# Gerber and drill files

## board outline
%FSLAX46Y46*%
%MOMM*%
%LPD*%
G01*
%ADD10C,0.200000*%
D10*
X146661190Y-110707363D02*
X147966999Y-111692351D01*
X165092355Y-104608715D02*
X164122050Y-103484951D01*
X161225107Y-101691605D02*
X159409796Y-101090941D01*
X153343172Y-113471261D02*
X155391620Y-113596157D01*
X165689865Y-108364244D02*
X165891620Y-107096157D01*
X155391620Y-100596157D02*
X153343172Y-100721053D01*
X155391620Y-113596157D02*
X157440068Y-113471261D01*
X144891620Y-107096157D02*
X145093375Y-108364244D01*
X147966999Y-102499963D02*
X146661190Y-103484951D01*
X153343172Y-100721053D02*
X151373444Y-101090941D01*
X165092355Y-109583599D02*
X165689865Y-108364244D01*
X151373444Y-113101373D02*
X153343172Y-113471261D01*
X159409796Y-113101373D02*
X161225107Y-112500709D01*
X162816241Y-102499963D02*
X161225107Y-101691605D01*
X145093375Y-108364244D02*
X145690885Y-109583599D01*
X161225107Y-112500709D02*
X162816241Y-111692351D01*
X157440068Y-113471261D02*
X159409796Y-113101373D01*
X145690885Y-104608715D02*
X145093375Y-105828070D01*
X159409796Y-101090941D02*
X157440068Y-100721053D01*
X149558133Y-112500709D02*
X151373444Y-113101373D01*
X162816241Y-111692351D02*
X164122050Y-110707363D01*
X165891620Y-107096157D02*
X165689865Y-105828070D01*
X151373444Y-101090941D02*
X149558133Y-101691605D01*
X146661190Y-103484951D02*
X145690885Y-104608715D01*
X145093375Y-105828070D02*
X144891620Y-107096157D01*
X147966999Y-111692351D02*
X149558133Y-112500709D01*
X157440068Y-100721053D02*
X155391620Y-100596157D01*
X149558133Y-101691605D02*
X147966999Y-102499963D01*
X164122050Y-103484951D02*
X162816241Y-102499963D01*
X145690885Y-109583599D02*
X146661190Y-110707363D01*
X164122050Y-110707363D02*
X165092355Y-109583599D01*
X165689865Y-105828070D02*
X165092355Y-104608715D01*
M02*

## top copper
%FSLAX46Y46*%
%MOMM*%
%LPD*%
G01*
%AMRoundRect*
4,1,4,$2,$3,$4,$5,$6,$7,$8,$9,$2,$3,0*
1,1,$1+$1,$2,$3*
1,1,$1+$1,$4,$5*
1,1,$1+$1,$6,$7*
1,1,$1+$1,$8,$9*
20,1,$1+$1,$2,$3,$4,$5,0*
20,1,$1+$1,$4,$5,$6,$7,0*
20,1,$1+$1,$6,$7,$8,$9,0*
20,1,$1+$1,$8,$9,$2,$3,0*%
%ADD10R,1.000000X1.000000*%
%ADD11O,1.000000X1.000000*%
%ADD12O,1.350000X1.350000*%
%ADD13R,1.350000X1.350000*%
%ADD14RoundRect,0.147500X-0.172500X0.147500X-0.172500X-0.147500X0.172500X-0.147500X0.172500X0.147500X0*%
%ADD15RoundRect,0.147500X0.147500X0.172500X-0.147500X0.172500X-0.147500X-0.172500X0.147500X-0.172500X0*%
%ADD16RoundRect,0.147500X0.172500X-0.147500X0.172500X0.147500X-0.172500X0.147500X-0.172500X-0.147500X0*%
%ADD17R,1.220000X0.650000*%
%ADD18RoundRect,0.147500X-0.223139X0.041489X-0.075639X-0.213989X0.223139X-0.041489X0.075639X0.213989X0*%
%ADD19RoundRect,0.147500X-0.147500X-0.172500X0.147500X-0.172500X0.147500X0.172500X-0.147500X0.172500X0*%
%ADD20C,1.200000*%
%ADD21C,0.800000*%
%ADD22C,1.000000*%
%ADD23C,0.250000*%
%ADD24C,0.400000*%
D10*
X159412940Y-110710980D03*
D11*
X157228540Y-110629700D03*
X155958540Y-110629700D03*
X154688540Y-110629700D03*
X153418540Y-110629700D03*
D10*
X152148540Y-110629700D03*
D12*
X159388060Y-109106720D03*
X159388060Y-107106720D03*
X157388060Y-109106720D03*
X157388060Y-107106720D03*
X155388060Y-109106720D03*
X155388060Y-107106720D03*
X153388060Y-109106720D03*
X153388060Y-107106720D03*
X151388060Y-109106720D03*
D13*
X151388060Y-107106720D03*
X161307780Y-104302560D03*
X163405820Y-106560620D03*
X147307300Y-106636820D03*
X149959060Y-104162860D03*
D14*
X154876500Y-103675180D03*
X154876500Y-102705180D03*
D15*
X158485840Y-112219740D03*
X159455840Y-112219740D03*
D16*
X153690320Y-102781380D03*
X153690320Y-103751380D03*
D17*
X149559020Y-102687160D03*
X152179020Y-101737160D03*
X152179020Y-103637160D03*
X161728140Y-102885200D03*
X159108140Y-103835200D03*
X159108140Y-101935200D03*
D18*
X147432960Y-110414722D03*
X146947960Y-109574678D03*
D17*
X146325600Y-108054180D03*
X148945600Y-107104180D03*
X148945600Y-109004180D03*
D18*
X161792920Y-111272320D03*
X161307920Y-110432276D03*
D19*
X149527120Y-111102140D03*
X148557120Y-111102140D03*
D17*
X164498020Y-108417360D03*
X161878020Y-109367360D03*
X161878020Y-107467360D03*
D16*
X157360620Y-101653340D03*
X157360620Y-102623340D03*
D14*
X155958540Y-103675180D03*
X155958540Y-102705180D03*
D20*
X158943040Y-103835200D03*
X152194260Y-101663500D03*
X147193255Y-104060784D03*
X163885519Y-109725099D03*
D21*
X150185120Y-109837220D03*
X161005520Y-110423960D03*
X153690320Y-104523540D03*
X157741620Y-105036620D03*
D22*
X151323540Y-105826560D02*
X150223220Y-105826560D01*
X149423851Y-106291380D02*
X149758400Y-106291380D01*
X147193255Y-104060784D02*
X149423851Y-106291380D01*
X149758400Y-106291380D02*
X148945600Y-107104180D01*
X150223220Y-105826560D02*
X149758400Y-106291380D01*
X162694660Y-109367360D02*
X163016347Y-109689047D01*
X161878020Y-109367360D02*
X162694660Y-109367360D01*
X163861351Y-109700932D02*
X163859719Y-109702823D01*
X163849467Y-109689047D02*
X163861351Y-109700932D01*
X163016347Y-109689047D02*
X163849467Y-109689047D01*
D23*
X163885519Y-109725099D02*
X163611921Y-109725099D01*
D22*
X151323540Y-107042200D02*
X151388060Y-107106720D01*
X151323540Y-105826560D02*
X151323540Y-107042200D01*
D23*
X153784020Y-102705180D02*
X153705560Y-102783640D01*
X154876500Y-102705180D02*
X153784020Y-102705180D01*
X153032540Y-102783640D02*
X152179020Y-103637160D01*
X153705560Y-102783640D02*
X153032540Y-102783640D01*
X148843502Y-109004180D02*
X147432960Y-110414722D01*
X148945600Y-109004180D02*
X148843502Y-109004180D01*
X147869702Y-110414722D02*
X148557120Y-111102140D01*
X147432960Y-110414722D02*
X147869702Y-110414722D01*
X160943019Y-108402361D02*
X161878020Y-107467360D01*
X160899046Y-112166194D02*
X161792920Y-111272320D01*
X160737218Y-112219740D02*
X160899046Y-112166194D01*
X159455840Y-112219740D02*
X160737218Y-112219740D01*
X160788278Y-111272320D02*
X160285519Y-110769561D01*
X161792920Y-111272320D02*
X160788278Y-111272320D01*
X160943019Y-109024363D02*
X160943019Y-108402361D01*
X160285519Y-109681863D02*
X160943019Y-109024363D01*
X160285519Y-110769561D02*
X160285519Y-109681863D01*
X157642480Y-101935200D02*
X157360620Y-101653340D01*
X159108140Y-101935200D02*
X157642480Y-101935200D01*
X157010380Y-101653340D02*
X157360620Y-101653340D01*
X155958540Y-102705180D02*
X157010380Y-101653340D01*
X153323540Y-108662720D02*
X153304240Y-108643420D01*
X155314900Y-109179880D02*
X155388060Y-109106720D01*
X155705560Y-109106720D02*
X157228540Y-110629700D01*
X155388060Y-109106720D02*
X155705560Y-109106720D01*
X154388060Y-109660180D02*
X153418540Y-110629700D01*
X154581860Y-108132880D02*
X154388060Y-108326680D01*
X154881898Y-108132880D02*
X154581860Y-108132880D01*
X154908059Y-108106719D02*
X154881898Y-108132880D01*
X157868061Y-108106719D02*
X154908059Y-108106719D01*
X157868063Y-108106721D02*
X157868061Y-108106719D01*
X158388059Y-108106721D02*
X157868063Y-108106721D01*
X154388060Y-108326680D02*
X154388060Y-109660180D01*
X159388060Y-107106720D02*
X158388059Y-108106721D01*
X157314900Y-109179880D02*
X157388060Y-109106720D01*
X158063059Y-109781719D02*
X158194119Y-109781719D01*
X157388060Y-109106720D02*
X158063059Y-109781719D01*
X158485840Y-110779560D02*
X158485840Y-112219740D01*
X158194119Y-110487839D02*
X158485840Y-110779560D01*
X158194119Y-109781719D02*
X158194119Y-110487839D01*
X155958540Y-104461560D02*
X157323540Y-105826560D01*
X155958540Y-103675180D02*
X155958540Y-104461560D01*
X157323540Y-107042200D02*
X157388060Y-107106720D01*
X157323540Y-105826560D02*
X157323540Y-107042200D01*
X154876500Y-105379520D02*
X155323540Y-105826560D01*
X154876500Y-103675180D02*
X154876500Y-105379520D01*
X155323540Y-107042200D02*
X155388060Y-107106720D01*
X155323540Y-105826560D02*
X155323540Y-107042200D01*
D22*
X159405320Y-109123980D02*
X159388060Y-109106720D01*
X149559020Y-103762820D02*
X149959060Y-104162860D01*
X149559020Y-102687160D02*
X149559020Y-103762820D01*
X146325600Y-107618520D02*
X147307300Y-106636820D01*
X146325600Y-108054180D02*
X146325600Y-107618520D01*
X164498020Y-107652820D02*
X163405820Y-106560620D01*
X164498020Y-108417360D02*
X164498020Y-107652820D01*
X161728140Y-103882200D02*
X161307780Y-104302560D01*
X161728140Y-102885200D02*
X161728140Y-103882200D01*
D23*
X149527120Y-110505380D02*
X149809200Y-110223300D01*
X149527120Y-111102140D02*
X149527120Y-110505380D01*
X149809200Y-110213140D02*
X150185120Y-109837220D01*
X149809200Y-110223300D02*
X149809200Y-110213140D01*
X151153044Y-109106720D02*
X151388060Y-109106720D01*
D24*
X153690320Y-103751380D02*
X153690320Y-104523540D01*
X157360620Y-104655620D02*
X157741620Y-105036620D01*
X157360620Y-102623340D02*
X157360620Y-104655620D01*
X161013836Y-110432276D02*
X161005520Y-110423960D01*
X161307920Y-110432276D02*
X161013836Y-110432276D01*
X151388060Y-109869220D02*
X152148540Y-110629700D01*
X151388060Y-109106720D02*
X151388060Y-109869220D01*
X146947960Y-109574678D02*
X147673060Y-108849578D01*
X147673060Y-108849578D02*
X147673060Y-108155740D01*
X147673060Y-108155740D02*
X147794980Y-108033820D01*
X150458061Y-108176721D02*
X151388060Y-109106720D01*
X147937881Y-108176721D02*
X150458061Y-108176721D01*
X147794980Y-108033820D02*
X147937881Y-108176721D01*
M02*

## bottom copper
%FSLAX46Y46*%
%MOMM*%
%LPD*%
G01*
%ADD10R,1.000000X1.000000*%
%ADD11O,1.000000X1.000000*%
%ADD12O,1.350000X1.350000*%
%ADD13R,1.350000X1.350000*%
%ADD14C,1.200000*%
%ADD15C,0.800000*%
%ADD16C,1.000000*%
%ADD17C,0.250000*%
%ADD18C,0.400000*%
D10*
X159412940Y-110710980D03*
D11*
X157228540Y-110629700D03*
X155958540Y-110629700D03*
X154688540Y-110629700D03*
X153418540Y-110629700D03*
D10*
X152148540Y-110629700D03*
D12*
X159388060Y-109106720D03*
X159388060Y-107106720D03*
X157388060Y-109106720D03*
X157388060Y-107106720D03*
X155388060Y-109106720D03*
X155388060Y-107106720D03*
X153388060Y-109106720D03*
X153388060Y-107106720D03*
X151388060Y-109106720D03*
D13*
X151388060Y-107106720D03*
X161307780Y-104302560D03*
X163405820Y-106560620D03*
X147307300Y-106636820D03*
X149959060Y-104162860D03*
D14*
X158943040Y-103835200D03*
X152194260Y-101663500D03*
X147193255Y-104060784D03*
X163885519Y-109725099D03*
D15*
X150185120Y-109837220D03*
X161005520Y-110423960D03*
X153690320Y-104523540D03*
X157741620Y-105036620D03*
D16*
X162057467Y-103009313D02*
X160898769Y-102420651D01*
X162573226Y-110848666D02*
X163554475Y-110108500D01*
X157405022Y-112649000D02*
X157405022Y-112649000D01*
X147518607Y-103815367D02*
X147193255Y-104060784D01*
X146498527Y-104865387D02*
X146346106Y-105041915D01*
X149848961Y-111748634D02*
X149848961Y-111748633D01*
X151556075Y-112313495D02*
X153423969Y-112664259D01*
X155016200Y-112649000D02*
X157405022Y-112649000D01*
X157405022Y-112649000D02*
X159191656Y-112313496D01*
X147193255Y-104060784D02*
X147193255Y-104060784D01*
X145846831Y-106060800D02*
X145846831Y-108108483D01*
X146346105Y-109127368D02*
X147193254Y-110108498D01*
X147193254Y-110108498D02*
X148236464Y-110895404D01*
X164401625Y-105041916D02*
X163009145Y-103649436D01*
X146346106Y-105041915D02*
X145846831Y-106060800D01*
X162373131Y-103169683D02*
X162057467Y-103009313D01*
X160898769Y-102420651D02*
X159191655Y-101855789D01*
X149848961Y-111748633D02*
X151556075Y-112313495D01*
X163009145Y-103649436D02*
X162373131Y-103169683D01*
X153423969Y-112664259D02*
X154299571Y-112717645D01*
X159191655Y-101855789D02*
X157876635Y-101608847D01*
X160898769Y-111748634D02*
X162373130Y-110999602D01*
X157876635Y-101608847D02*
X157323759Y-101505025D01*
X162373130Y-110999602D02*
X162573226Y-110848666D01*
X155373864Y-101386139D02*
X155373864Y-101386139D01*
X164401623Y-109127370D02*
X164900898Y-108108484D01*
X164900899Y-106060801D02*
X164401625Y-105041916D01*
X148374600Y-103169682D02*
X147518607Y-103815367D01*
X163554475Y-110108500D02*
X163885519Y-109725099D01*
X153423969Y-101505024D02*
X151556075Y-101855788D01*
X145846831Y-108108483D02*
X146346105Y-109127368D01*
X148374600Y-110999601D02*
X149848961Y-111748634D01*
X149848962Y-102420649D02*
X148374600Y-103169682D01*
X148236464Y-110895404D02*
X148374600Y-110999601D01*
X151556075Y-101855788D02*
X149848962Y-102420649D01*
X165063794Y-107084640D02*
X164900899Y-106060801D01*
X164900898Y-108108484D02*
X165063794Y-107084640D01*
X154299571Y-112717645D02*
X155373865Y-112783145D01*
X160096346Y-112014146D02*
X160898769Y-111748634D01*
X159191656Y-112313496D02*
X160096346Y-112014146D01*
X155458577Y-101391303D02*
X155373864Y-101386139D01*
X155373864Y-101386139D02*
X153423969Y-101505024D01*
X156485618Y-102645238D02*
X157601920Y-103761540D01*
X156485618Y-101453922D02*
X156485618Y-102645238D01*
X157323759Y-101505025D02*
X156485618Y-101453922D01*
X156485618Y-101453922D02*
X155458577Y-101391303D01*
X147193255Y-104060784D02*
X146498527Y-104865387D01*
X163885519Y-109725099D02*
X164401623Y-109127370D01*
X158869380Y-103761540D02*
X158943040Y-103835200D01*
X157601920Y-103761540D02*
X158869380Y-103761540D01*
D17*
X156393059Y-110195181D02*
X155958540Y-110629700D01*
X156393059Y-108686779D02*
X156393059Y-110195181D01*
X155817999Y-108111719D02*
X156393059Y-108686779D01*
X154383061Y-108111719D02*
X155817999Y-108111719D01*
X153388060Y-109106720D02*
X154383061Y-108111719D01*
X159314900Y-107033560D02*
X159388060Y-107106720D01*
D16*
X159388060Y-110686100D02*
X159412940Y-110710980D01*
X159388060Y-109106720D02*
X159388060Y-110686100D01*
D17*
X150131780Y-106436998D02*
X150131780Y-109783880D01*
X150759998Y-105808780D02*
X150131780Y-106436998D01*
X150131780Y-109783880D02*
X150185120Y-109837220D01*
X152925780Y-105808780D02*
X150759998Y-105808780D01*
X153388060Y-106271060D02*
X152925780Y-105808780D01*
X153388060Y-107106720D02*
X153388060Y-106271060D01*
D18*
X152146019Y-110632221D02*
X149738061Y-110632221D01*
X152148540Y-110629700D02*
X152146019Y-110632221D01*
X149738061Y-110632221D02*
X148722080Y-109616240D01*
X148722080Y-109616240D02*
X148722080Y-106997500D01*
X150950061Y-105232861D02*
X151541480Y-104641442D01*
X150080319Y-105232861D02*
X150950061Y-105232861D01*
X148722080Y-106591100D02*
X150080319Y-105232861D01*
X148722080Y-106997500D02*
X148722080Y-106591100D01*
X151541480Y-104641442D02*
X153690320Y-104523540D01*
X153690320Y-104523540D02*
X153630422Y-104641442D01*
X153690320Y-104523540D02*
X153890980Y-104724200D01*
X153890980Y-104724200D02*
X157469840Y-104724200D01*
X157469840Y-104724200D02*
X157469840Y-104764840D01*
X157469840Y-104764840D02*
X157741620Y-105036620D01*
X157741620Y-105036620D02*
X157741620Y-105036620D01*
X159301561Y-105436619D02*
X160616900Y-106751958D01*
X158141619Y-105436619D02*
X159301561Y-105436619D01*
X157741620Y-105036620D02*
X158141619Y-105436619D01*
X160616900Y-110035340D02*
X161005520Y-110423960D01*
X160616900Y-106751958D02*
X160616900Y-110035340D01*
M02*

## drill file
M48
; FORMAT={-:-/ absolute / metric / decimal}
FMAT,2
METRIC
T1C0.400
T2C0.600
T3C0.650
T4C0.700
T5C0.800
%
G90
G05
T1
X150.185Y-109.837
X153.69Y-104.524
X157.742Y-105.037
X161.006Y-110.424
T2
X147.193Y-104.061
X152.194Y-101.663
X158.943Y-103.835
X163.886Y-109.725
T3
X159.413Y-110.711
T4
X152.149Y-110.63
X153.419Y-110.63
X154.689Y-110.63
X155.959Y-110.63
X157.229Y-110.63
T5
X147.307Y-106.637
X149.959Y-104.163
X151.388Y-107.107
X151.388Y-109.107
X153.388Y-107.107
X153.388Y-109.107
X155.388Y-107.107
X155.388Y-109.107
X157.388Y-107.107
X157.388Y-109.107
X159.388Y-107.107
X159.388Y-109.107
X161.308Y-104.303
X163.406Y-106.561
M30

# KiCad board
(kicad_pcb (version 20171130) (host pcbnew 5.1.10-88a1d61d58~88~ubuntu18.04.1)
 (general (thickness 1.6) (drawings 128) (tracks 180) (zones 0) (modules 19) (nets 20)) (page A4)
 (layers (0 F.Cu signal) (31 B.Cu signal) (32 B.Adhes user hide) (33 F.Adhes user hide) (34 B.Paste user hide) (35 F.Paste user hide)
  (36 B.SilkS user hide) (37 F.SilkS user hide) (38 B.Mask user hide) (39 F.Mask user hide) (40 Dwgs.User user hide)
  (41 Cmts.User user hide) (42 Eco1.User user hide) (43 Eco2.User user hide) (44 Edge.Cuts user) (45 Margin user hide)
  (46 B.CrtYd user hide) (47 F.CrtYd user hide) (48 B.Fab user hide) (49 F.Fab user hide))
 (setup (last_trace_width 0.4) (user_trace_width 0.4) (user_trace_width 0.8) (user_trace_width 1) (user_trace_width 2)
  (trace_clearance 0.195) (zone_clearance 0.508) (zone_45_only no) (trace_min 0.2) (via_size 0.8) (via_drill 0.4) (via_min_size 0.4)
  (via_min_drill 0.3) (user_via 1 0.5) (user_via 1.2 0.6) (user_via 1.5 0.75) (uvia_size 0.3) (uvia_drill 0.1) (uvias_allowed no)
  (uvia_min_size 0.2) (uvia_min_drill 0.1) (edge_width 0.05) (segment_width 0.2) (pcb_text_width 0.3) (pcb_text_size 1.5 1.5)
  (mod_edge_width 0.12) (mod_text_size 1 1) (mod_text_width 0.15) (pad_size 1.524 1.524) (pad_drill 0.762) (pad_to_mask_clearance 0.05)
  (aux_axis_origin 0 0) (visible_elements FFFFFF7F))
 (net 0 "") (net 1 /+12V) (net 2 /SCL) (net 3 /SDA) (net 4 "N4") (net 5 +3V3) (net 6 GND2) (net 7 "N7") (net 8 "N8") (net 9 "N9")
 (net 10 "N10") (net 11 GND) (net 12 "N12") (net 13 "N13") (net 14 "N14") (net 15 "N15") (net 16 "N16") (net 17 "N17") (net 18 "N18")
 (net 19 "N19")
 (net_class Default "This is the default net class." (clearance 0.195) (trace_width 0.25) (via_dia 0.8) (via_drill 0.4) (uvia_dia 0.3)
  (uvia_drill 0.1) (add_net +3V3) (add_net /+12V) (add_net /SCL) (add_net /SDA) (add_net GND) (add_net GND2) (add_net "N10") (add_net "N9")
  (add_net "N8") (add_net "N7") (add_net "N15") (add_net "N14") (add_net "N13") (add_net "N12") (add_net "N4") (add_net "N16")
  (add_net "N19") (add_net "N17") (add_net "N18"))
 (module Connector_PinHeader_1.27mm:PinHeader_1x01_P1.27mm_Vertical (layer F.Cu) (at 159.41294 110.71098)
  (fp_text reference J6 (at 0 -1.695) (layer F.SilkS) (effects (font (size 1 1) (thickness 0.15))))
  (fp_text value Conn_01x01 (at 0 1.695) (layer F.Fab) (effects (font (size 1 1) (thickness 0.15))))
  (pad 1 thru_hole rect (at 0 0) (size 1 1) (drill 0.65) (layers *.Cu *.Mask) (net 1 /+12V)))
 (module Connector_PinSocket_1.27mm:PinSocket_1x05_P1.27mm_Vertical (layer F.Cu) (at 152.14854 110.6297 90)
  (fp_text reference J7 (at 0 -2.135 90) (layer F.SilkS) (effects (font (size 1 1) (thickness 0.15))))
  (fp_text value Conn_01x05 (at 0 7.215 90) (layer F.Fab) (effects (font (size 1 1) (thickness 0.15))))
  (pad 5 thru_hole oval (at 0 5.08 90) (size 1 1) (drill 0.7) (layers *.Cu *.Mask) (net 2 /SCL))
  (pad 4 thru_hole oval (at 0 3.81 90) (size 1 1) (drill 0.7) (layers *.Cu *.Mask) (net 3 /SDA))
  (pad 3 thru_hole oval (at 0 2.54 90) (size 1 1) (drill 0.7) (layers *.Cu *.Mask) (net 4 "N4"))
  (pad 2 thru_hole oval (at 0 1.27 90) (size 1 1) (drill 0.7) (layers *.Cu *.Mask) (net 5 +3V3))
  (pad 1 thru_hole rect (at 0 0 90) (size 1 1) (drill 0.7) (layers *.Cu *.Mask) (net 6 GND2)))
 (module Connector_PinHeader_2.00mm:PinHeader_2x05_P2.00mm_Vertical (layer B.Cu) (at 151.38806 107.10672 270)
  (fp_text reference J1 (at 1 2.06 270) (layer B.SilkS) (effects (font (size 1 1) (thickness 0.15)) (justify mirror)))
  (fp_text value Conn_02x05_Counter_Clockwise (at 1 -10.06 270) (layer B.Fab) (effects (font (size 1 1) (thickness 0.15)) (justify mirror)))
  (pad 10 thru_hole oval (at 2 -8 270) (size 1.35 1.35) (drill 0.8) (layers *.Cu *.Mask) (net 1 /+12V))
  (pad 9 thru_hole oval (at 0 -8 270) (size 1.35 1.35) (drill 0.8) (layers *.Cu *.Mask) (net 5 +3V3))
  (pad 8 thru_hole oval (at 2 -6 270) (size 1.35 1.35) (drill 0.8) (layers *.Cu *.Mask) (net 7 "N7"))
  (pad 7 thru_hole oval (at 0 -6 270) (size 1.35 1.35) (drill 0.8) (layers *.Cu *.Mask) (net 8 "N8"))
  (pad 6 thru_hole oval (at 2 -4 270) (size 1.35 1.35) (drill 0.8) (layers *.Cu *.Mask) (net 2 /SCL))
  (pad 5 thru_hole oval (at 0 -4 270) (size 1.35 1.35) (drill 0.8) (layers *.Cu *.Mask) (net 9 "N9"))
  (pad 4 thru_hole oval (at 2 -2 270) (size 1.35 1.35) (drill 0.8) (layers *.Cu *.Mask) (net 3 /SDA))
  (pad 3 thru_hole oval (at 0 -2 270) (size 1.35 1.35) (drill 0.8) (layers *.Cu *.Mask) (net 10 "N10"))
  (pad 2 thru_hole oval (at 2 0 270) (size 1.35 1.35) (drill 0.8) (layers *.Cu *.Mask) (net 6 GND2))
  (pad 1 thru_hole rect (at 0 0 270) (size 1.35 1.35) (drill 0.8) (layers *.Cu *.Mask) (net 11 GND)))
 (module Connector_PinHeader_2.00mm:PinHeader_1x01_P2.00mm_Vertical (layer F.Cu) (at 161.30778 104.30256)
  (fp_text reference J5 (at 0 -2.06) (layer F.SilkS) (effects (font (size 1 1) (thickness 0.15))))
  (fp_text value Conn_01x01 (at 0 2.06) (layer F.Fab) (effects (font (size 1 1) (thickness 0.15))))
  (pad 1 thru_hole rect (at 0 0) (size 1.35 1.35) (drill 0.8) (layers *.Cu *.Mask) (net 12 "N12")))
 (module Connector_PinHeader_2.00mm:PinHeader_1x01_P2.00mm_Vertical (layer F.Cu) (at 163.40582 106.56062)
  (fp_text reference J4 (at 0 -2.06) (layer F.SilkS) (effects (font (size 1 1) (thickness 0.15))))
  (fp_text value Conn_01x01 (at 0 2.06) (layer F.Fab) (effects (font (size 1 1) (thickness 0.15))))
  (pad 1 thru_hole rect (at 0 0) (size 1.35 1.35) (drill 0.8) (layers *.Cu *.Mask) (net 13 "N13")))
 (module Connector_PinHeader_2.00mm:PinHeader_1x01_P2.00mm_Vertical (layer F.Cu) (at 147.3073 106.63682)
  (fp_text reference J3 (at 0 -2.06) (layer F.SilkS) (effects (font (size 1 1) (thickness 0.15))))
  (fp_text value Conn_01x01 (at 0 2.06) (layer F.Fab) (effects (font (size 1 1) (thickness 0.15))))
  (pad 1 thru_hole rect (at 0 0) (size 1.35 1.35) (drill 0.8) (layers *.Cu *.Mask) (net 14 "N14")))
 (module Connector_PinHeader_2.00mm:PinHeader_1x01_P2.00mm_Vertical (layer F.Cu) (at 149.95906 104.16286)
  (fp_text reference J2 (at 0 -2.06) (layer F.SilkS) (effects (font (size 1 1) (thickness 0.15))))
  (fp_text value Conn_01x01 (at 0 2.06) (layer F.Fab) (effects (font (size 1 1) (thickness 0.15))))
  (pad 1 thru_hole rect (at 0 0) (size 1.35 1.35) (drill 0.8) (layers *.Cu *.Mask) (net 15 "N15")))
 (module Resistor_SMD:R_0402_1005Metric (layer F.Cu) (at 154.8765 103.19018 270)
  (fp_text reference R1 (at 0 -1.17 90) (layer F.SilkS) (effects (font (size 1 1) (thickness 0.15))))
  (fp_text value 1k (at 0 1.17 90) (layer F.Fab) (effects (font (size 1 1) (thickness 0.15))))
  (pad 2 smd roundrect (at 0.485 0 270) (size 0.59 0.64) (layers F.Cu F.Paste F.Mask) (roundrect_rratio 0.25) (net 9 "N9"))
  (pad 1 smd roundrect (at -0.485 0 270) (size 0.59 0.64) (layers F.Cu F.Paste F.Mask) (roundrect_rratio 0.25) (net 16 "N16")))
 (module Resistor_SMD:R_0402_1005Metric (layer F.Cu) (at 158.97084 112.21974 180)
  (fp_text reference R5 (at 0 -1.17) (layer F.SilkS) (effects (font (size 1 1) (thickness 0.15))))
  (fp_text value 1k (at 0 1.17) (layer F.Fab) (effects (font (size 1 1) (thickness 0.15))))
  (pad 2 smd roundrect (at 0.485 0 180) (size 0.59 0.64) (layers F.Cu F.Paste F.Mask) (roundrect_rratio 0.25) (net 7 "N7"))
  (pad 1 smd roundrect (at -0.485 0 180) (size 0.59 0.64) (layers F.Cu F.Paste F.Mask) (roundrect_rratio 0.25) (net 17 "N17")))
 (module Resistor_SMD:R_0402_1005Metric (layer F.Cu) (at 153.69032 103.26638 90)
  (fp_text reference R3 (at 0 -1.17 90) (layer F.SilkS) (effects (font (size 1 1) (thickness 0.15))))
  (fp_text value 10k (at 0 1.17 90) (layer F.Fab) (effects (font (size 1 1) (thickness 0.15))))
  (pad 2 smd roundrect (at 0.485 0 90) (size 0.59 0.64) (layers F.Cu F.Paste F.Mask) (roundrect_rratio 0.25) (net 16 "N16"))
  (pad 1 smd roundrect (at -0.485 0 90) (size 0.59 0.64) (layers F.Cu F.Paste F.Mask) (roundrect_rratio 0.25) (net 6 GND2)))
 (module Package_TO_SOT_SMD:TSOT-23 (layer F.Cu) (at 150.86902 102.68716 180)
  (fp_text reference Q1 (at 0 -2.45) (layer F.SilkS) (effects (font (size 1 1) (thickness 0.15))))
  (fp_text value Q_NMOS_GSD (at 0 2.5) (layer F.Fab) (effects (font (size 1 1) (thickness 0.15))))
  (pad 3 smd rect (at 1.31 0 180) (size 1.22 0.65) (layers F.Cu F.Paste F.Mask) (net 15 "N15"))
  (pad 2 smd rect (at -1.31 0.95 180) (size 1.22 0.65) (layers F.Cu F.Paste F.Mask) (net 11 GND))
  (pad 1 smd rect (at -1.31 -0.95 180) (size 1.22 0.65) (layers F.Cu F.Paste F.Mask) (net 16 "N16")))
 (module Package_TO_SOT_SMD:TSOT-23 (layer F.Cu) (at 160.41814 102.8852)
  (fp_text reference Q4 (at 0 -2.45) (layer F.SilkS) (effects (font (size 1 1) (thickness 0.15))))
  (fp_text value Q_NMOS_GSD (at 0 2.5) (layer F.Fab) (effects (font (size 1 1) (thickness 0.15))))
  (pad 3 smd rect (at 1.31 0) (size 1.22 0.65) (layers F.Cu F.Paste F.Mask) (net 12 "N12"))
  (pad 2 smd rect (at -1.31 0.95) (size 1.22 0.65) (layers F.Cu F.Paste F.Mask) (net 11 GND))
  (pad 1 smd rect (at -1.31 -0.95) (size 1.22 0.65) (layers F.Cu F.Paste F.Mask) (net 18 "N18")))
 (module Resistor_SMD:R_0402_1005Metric (layer F.Cu) (at 147.19046 109.9947 300)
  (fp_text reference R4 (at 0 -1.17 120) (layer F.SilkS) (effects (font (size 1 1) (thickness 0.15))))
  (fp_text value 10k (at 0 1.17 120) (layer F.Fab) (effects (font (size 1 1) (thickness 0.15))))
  (pad 2 smd roundrect (at 0.485 0 300) (size 0.59 0.64) (layers F.Cu F.Paste F.Mask) (roundrect_rratio 0.25) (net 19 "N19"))
  (pad 1 smd roundrect (at -0.485 0 300) (size 0.59 0.64) (layers F.Cu F.Paste F.Mask) (roundrect_rratio 0.25) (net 6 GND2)))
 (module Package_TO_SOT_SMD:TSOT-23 (layer F.Cu) (at 147.6356 108.05418 180)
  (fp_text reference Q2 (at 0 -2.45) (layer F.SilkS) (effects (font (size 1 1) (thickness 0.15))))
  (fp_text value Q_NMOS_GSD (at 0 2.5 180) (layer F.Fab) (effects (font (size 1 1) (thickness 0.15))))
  (pad 3 smd rect (at 1.31 0 180) (size 1.22 0.65) (layers F.Cu F.Paste F.Mask) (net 14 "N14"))
  (pad 2 smd rect (at -1.31 0.95 180) (size 1.22 0.65) (layers F.Cu F.Paste F.Mask) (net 11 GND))
  (pad 1 smd rect (at -1.31 -0.95 180) (size 1.22 0.65) (layers F.Cu F.Paste F.Mask) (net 19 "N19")))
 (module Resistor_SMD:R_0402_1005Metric (layer F.Cu) (at 161.55042 110.852298 300)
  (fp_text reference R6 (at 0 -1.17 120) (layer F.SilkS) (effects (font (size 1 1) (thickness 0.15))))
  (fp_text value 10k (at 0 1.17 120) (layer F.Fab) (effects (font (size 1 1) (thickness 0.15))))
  (pad 2 smd roundrect (at 0.485 0 300) (size 0.59 0.64) (layers F.Cu F.Paste F.Mask) (roundrect_rratio 0.25) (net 17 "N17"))
  (pad 1 smd roundrect (at -0.485 0 300) (size 0.59 0.64) (layers F.Cu F.Paste F.Mask) (roundrect_rratio 0.25) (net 6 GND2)))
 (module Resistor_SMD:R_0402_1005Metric (layer F.Cu) (at 149.04212 111.10214)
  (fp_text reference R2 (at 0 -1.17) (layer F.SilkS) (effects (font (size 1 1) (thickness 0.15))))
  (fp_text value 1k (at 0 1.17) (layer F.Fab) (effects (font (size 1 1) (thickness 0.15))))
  (pad 2 smd roundrect (at 0.485 0) (size 0.59 0.64) (layers F.Cu F.Paste F.Mask) (roundrect_rratio 0.25) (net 10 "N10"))
  (pad 1 smd roundrect (at -0.485 0) (size 0.59 0.64) (layers F.Cu F.Paste F.Mask) (roundrect_rratio 0.25) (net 19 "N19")))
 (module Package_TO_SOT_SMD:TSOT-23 (layer F.Cu) (at 163.18802 108.41736)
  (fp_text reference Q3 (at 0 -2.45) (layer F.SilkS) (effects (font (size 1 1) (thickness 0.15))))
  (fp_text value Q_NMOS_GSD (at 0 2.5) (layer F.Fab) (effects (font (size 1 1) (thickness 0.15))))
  (pad 3 smd rect (at 1.31 0) (size 1.22 0.65) (layers F.Cu F.Paste F.Mask) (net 13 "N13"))
  (pad 2 smd rect (at -1.31 0.95) (size 1.22 0.65) (layers F.Cu F.Paste F.Mask) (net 11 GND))
  (pad 1 smd rect (at -1.31 -0.95) (size 1.22 0.65) (layers F.Cu F.Paste F.Mask) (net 17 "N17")))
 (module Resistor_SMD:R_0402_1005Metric (layer F.Cu) (at 157.36062 102.13834 90)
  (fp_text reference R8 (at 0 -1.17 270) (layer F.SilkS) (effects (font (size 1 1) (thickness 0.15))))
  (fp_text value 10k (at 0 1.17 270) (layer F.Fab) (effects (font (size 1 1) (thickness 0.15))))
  (pad 2 smd roundrect (at 0.485 0 90) (size 0.59 0.64) (layers F.Cu F.Paste F.Mask) (roundrect_rratio 0.25) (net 18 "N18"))
  (pad 1 smd roundrect (at -0.485 0 90) (size 0.59 0.64) (layers F.Cu F.Paste F.Mask) (roundrect_rratio 0.25) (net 6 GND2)))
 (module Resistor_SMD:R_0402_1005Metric (layer F.Cu) (at 155.95854 103.19018 270)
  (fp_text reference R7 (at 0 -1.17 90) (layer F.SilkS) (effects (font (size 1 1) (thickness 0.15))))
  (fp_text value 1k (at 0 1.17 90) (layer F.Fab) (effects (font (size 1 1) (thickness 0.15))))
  (pad 2 smd roundrect (at 0.485 0 270) (size 0.59 0.64) (layers F.Cu F.Paste F.Mask) (roundrect_rratio 0.25) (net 8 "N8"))
  (pad 1 smd roundrect (at -0.485 0 270) (size 0.59 0.64) (layers F.Cu F.Paste F.Mask) (roundrect_rratio 0.25) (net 18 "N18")))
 (gr_line (start 146.66119 110.707363) (end 147.966999 111.692351) (layer Edge.Cuts) (width 0.2))
 (gr_line (start 165.092355 104.608715) (end 164.12205 103.484951) (layer Edge.Cuts) (width 0.2))
 (gr_line (start 161.225107 101.691605) (end 159.409796 101.090941) (layer Edge.Cuts) (width 0.2))
 (gr_line (start 153.343172 113.471261) (end 155.39162 113.596157) (layer Edge.Cuts) (width 0.2))
 (gr_line (start 165.689865 108.364244) (end 165.89162 107.096157) (layer Edge.Cuts) (width 0.2))
 (gr_line (start 155.39162 100.596157) (end 153.343172 100.721053) (layer Edge.Cuts) (width 0.2))
 (gr_line (start 155.39162 113.596157) (end 157.440068 113.471261) (layer Edge.Cuts) (width 0.2))
 (gr_line (start 144.89162 107.096157) (end 145.093375 108.364244) (layer Edge.Cuts) (width 0.2))
 (gr_line (start 147.966999 102.499963) (end 146.66119 103.484951) (layer Edge.Cuts) (width 0.2))
 (gr_line (start 153.343172 100.721053) (end 151.373444 101.090941) (layer Edge.Cuts) (width 0.2))
 (gr_line (start 165.092355 109.583599) (end 165.689865 108.364244) (layer Edge.Cuts) (width 0.2))
 (gr_line (start 151.373444 113.101373) (end 153.343172 113.471261) (layer Edge.Cuts) (width 0.2))
 (gr_line (start 159.409796 113.101373) (end 161.225107 112.500709) (layer Edge.Cuts) (width 0.2))
 (gr_line (start 162.816241 102.499963) (end 161.225107 101.691605) (layer Edge.Cuts) (width 0.2))
 (gr_line (start 145.093375 108.364244) (end 145.690885 109.583599) (layer Edge.Cuts) (width 0.2))
 (gr_line (start 161.225107 112.500709) (end 162.816241 111.692351) (layer Edge.Cuts) (width 0.2))
 (gr_line (start 157.440068 113.471261) (end 159.409796 113.101373) (layer Edge.Cuts) (width 0.2))
 (gr_line (start 145.690885 104.608715) (end 145.093375 105.82807) (layer Edge.Cuts) (width 0.2))
 (gr_line (start 159.409796 101.090941) (end 157.440068 100.721053) (layer Edge.Cuts) (width 0.2))
 (gr_line (start 149.558133 112.500709) (end 151.373444 113.101373) (layer Edge.Cuts) (width 0.2))
 (gr_line (start 162.816241 111.692351) (end 164.12205 110.707363) (layer Edge.Cuts) (width 0.2))
 (gr_line (start 165.89162 107.096157) (end 165.689865 105.82807) (layer Edge.Cuts) (width 0.2))
 (gr_line (start 151.373444 101.090941) (end 149.558133 101.691605) (layer Edge.Cuts) (width 0.2))
 (gr_line (start 146.66119 103.484951) (end 145.690885 104.608715) (layer Edge.Cuts) (width 0.2))
 (gr_line (start 145.093375 105.82807) (end 144.89162 107.096157) (layer Edge.Cuts) (width 0.2))
 (gr_line (start 147.966999 111.692351) (end 149.558133 112.500709) (layer Edge.Cuts) (width 0.2))
 (gr_line (start 157.440068 100.721053) (end 155.39162 100.596157) (layer Edge.Cuts) (width 0.2))
 (gr_line (start 149.558133 101.691605) (end 147.966999 102.499963) (layer Edge.Cuts) (width 0.2))
 (gr_line (start 164.12205 103.484951) (end 162.816241 102.499963) (layer Edge.Cuts) (width 0.2))
 (gr_line (start 145.690885 109.583599) (end 146.66119 110.707363) (layer Edge.Cuts) (width 0.2))
 (gr_line (start 164.12205 110.707363) (end 165.092355 109.583599) (layer Edge.Cuts) (width 0.2))
 (gr_line (start 165.689865 105.82807) (end 165.092355 104.608715) (layer Edge.Cuts) (width 0.2))
 (segment (start 162.057467 103.009313) (end 160.898769 102.420651) (width 1) (layer B.Cu) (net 11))
 (segment (start 162.573226 110.848666) (end 163.554475 110.1085) (width 1) (layer B.Cu) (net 11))
 (segment (start 157.405022 112.649) (end 157.405022 112.649) (width 1) (layer B.Cu) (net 11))
 (segment (start 147.518607 103.815367) (end 147.193255 104.060784) (width 1) (layer B.Cu) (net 11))
 (segment (start 146.498527 104.865387) (end 146.346106 105.041915) (width 1) (layer B.Cu) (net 11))
 (segment (start 149.848961 111.748634) (end 149.848961 111.748633) (width 1) (layer B.Cu) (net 11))
 (segment (start 151.556075 112.313495) (end 153.423969 112.664259) (width 1) (layer B.Cu) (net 11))
 (segment (start 155.0162 112.649) (end 157.405022 112.649) (width 1) (layer B.Cu) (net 11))
 (segment (start 157.405022 112.649) (end 159.191656 112.313496) (width 1) (layer B.Cu) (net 11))
 (segment (start 147.193255 104.060784) (end 147.193255 104.060784) (width 1) (layer B.Cu) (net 11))
 (segment (start 145.846831 106.0608) (end 145.846831 108.108483) (width 1) (layer B.Cu) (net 11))
 (segment (start 146.346105 109.127368) (end 147.193254 110.108498) (width 1) (layer B.Cu) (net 11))
 (segment (start 147.193254 110.108498) (end 148.236464 110.895404) (width 1) (layer B.Cu) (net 11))
 (segment (start 164.401625 105.041916) (end 163.009145 103.649436) (width 1) (layer B.Cu) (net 11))
 (segment (start 146.346106 105.041915) (end 145.846831 106.0608) (width 1) (layer B.Cu) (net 11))
 (segment (start 162.373131 103.169683) (end 162.057467 103.009313) (width 1) (layer B.Cu) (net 11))
 (segment (start 160.898769 102.420651) (end 159.191655 101.855789) (width 1) (layer B.Cu) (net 11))
 (segment (start 149.848961 111.748633) (end 151.556075 112.313495) (width 1) (layer B.Cu) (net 11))
 (segment (start 163.009145 103.649436) (end 162.373131 103.169683) (width 1) (layer B.Cu) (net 11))
 (segment (start 153.423969 112.664259) (end 154.299571 112.717645) (width 1) (layer B.Cu) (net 11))
 (segment (start 159.191655 101.855789) (end 157.876635 101.608847) (width 1) (layer B.Cu) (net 11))
 (segment (start 160.898769 111.748634) (end 162.37313 110.999602) (width 1) (layer B.Cu) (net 11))
 (segment (start 157.876635 101.608847) (end 157.323759 101.505025) (width 1) (layer B.Cu) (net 11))
 (segment (start 162.37313 110.999602) (end 162.573226 110.848666) (width 1) (layer B.Cu) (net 11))
 (segment (start 155.373864 101.386139) (end 155.373864 101.386139) (width 1) (layer B.Cu) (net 11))
 (segment (start 164.401623 109.12737) (end 164.900898 108.108484) (width 1) (layer B.Cu) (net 11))
 (segment (start 164.900899 106.060801) (end 164.401625 105.041916) (width 1) (layer B.Cu) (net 11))
 (segment (start 148.3746 103.169682) (end 147.518607 103.815367) (width 1) (layer B.Cu) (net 11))
 (segment (start 163.554475 110.1085) (end 163.885519 109.725099) (width 1) (layer B.Cu) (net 11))
 (segment (start 153.423969 101.505024) (end 151.556075 101.855788) (width 1) (layer B.Cu) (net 11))
 (segment (start 145.846831 108.108483) (end 146.346105 109.127368) (width 1) (layer B.Cu) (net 11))
 (segment (start 148.3746 110.999601) (end 149.848961 111.748634) (width 1) (layer B.Cu) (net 11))
 (segment (start 149.848962 102.420649) (end 148.3746 103.169682) (width 1) (layer B.Cu) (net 11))
 (segment (start 148.236464 110.895404) (end 148.3746 110.999601) (width 1) (layer B.Cu) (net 11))
 (segment (start 151.556075 101.855788) (end 149.848962 102.420649) (width 1) (layer B.Cu) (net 11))
 (segment (start 165.063794 107.08464) (end 164.900899 106.060801) (width 1) (layer B.Cu) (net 11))
 (segment (start 164.900898 108.108484) (end 165.063794 107.08464) (width 1) (layer B.Cu) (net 11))
 (segment (start 154.299571 112.717645) (end 155.373865 112.783145) (width 1) (layer B.Cu) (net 11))
 (segment (start 160.096346 112.014146) (end 160.898769 111.748634) (width 1) (layer B.Cu) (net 11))
 (segment (start 159.191656 112.313496) (end 160.096346 112.014146) (width 1) (layer B.Cu) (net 11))
 (segment (start 155.458577 101.391303) (end 155.373864 101.386139) (width 1) (layer B.Cu) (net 11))
 (via (at 158.94304 103.8352) (size 1.2) (drill 0.6) (layers F.Cu B.Cu) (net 11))
 (segment (start 155.373864 101.386139) (end 153.423969 101.505024) (width 1) (layer B.Cu) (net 11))
 (via (at 152.19426 101.6635) (size 1.2) (drill 0.6) (layers F.Cu B.Cu) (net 11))
 (segment (start 156.485618 102.645238) (end 157.60192 103.76154) (width 1) (layer B.Cu) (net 11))
 (segment (start 156.485618 101.453922) (end 156.485618 102.645238) (width 1) (layer B.Cu) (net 11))
 (segment (start 157.323759 101.505025) (end 156.485618 101.453922) (width 1) (layer B.Cu) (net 11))
 (segment (start 156.485618 101.453922) (end 155.458577 101.391303) (width 1) (layer B.Cu) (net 11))
 (segment (start 151.32354 105.82656) (end 150.22322 105.82656) (width 1) (layer F.Cu) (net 11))
 (segment (start 147.193255 104.060784) (end 146.498527 104.865387) (width 1) (layer B.Cu) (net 11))
 (via (at 147.193255 104.060784) (size 1.2) (drill 0.6) (layers F.Cu B.Cu) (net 11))
 (segment (start 149.423851 106.29138) (end 149.7584 106.29138) (width 1) (layer F.Cu) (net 11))
 (segment (start 147.193255 104.060784) (end 149.423851 106.29138) (width 1) (layer F.Cu) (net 11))
 (segment (start 149.7584 106.29138) (end 148.9456 107.10418) (width 1) (layer F.Cu) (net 11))
 (segment (start 150.22322 105.82656) (end 149.7584 106.29138) (width 1) (layer F.Cu) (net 11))
 (segment (start 163.885519 109.725099) (end 164.401623 109.12737) (width 1) (layer B.Cu) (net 11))
 (via (at 163.885519 109.725099) (size 1.2) (drill 0.6) (layers F.Cu B.Cu) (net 11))
 (segment (start 162.69466 109.36736) (end 163.016347 109.689047) (width 1) (layer F.Cu) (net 11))
 (segment (start 161.87802 109.36736) (end 162.69466 109.36736) (width 1) (layer F.Cu) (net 11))
 (segment (start 163.861351 109.700932) (end 163.859719 109.702823) (width 1) (layer F.Cu) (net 11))
 (segment (start 163.849467 109.689047) (end 163.861351 109.700932) (width 1) (layer F.Cu) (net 11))
 (segment (start 163.016347 109.689047) (end 163.849467 109.689047) (width 1) (layer F.Cu) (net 11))
 (segment (start 163.885519 109.725099) (end 163.611921 109.725099) (width 0.25) (layer F.Cu) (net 11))
 (segment (start 151.32354 107.0422) (end 151.38806 107.10672) (width 1) (layer F.Cu) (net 11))
 (segment (start 151.32354 105.82656) (end 151.32354 107.0422) (width 1) (layer F.Cu) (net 11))
 (segment (start 158.86938 103.76154) (end 158.94304 103.8352) (width 1) (layer B.Cu) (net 11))
 (segment (start 157.60192 103.76154) (end 158.86938 103.76154) (width 1) (layer B.Cu) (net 11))
 (segment (start 153.78402 102.70518) (end 153.70556 102.78364) (width 0.25) (layer F.Cu) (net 16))
 (segment (start 154.8765 102.70518) (end 153.78402 102.70518) (width 0.25) (layer F.Cu) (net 16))
 (segment (start 153.03254 102.78364) (end 152.17902 103.63716) (width 0.25) (layer F.Cu) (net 16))
 (segment (start 153.70556 102.78364) (end 153.03254 102.78364) (width 0.25) (layer F.Cu) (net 16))
 (segment (start 148.843502 109.00418) (end 147.43296 110.414722) (width 0.25) (layer F.Cu) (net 19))
 (segment (start 148.9456 109.00418) (end 148.843502 109.00418) (width 0.25) (layer F.Cu) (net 19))
 (segment (start 147.869702 110.414722) (end 148.55712 111.10214) (width 0.25) (layer F.Cu) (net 19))
 (segment (start 147.43296 110.414722) (end 147.869702 110.414722) (width 0.25) (layer F.Cu) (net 19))
 (segment (start 160.943019 108.402361) (end 161.87802 107.46736) (width 0.25) (layer F.Cu) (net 17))
 (segment (start 160.899046 112.166194) (end 161.79292 111.27232) (width 0.25) (layer F.Cu) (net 17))
 (segment (start 160.737218 112.21974) (end 160.899046 112.166194) (width 0.25) (layer F.Cu) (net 17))
 (segment (start 159.45584 112.21974) (end 160.737218 112.21974) (width 0.25) (layer F.Cu) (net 17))
 (segment (start 160.788278 111.27232) (end 160.285519 110.769561) (width 0.25) (layer F.Cu) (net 17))
 (segment (start 161.79292 111.27232) (end 160.788278 111.27232) (width 0.25) (layer F.Cu) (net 17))
 (segment (start 160.943019 109.024363) (end 160.943019 108.402361) (width 0.25) (layer F.Cu) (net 17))
 (segment (start 160.285519 109.681863) (end 160.943019 109.024363) (width 0.25) (layer F.Cu) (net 17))
 (segment (start 160.285519 110.769561) (end 160.285519 109.681863) (width 0.25) (layer F.Cu) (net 17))
 (segment (start 157.64248 101.9352) (end 157.36062 101.65334) (width 0.25) (layer F.Cu) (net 18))
 (segment (start 159.10814 101.9352) (end 157.64248 101.9352) (width 0.25) (layer F.Cu) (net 18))
 (segment (start 157.01038 101.65334) (end 157.36062 101.65334) (width 0.25) (layer F.Cu) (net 18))
 (segment (start 155.95854 102.70518) (end 157.01038 101.65334) (width 0.25) (layer F.Cu) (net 18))
 (segment (start 153.32354 108.66272) (end 153.30424 108.64342) (width 0.25) (layer F.Cu) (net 3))
 (segment (start 156.393059 110.195181) (end 155.95854 110.6297) (width 0.25) (layer B.Cu) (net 3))
 (segment (start 156.393059 108.686779) (end 156.393059 110.195181) (width 0.25) (layer B.Cu) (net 3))
 (segment (start 155.817999 108.111719) (end 156.393059 108.686779) (width 0.25) (layer B.Cu) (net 3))
 (segment (start 154.383061 108.111719) (end 155.817999 108.111719) (width 0.25) (layer B.Cu) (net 3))
 (segment (start 153.38806 109.10672) (end 154.383061 108.111719) (width 0.25) (layer B.Cu) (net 3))
 (segment (start 155.3149 109.17988) (end 155.38806 109.10672) (width 0.25) (layer F.Cu) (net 2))
 (segment (start 155.70556 109.10672) (end 157.22854 110.6297) (width 0.25) (layer F.Cu) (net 2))
 (segment (start 155.38806 109.10672) (end 155.70556 109.10672) (width 0.25) (layer F.Cu) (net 2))
 (segment (start 159.3149 107.03356) (end 159.38806 107.10672) (width 0.25) (layer B.Cu) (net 5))
 (segment (start 154.38806 109.66018) (end 153.41854 110.6297) (width 0.25) (layer F.Cu) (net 5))
 (segment (start 154.58186 108.13288) (end 154.38806 108.32668) (width 0.25) (layer F.Cu) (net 5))
 (segment (start 154.881898 108.13288) (end 154.58186 108.13288) (width 0.25) (layer F.Cu) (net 5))
 (segment (start 154.908059 108.106719) (end 154.881898 108.13288) (width 0.25) (layer F.Cu) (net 5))
 (segment (start 157.868061 108.106719) (end 154.908059 108.106719) (width 0.25) (layer F.Cu) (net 5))
 (segment (start 157.868063 108.106721) (end 157.868061 108.106719) (width 0.25) (layer F.Cu) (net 5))
 (segment (start 158.388059 108.106721) (end 157.868063 108.106721) (width 0.25) (layer F.Cu) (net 5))
 (segment (start 154.38806 108.32668) (end 154.38806 109.66018) (width 0.25) (layer F.Cu) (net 5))
 (segment (start 159.38806 107.10672) (end 158.388059 108.106721) (width 0.25) (layer F.Cu) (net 5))
 (segment (start 157.3149 109.17988) (end 157.38806 109.10672) (width 0.25) (layer F.Cu) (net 7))
 (segment (start 158.063059 109.781719) (end 158.194119 109.781719) (width 0.25) (layer F.Cu) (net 7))
 (segment (start 157.38806 109.10672) (end 158.063059 109.781719) (width 0.25) (layer F.Cu) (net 7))
 (segment (start 158.48584 110.77956) (end 158.48584 112.21974) (width 0.25) (layer F.Cu) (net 7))
 (segment (start 158.194119 110.487839) (end 158.48584 110.77956) (width 0.25) (layer F.Cu) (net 7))
 (segment (start 158.194119 109.781719) (end 158.194119 110.487839) (width 0.25) (layer F.Cu) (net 7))
 (segment (start 155.95854 104.46156) (end 157.32354 105.82656) (width 0.25) (layer F.Cu) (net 8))
 (segment (start 155.95854 103.67518) (end 155.95854 104.46156) (width 0.25) (layer F.Cu) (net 8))
 (segment (start 157.32354 107.0422) (end 157.38806 107.10672) (width 0.25) (layer F.Cu) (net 8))
 (segment (start 157.32354 105.82656) (end 157.32354 107.0422) (width 0.25) (layer F.Cu) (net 8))
 (segment (start 154.8765 105.37952) (end 155.32354 105.82656) (width 0.25) (layer F.Cu) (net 9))
 (segment (start 154.8765 103.67518) (end 154.8765 105.37952) (width 0.25) (layer F.Cu) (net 9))
 (segment (start 155.32354 107.0422) (end 155.38806 107.10672) (width 0.25) (layer F.Cu) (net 9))
 (segment (start 155.32354 105.82656) (end 155.32354 107.0422) (width 0.25) (layer F.Cu) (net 9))
 (segment (start 159.40532 109.12398) (end 159.38806 109.10672) (width 1) (layer F.Cu) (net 1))
 (segment (start 159.38806 110.6861) (end 159.41294 110.71098) (width 1) (layer B.Cu) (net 1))
 (segment (start 159.38806 109.10672) (end 159.38806 110.6861) (width 1) (layer B.Cu) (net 1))
 (segment (start 149.55902 103.76282) (end 149.95906 104.16286) (width 1) (layer F.Cu) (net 15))
 (segment (start 149.55902 102.68716) (end 149.55902 103.76282) (width 1) (layer F.Cu) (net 15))
 (segment (start 146.3256 107.61852) (end 147.3073 106.63682) (width 1) (layer F.Cu) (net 14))
 (segment (start 146.3256 108.05418) (end 146.3256 107.61852) (width 1) (layer F.Cu) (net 14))
 (segment (start 164.49802 107.65282) (end 163.40582 106.56062) (width 1) (layer F.Cu) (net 13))
 (segment (start 164.49802 108.41736) (end 164.49802 107.65282) (width 1) (layer F.Cu) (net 13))
 (segment (start 161.72814 103.8822) (end 161.30778 104.30256) (width 1) (layer F.Cu) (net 12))
 (segment (start 161.72814 102.8852) (end 161.72814 103.8822) (width 1) (layer F.Cu) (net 12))
 (via (at 150.18512 109.83722) (size 0.8) (drill 0.4) (layers F.Cu B.Cu) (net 10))
 (segment (start 149.52712 110.50538) (end 149.8092 110.2233) (width 0.25) (layer F.Cu) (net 10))
 (segment (start 149.52712 111.10214) (end 149.52712 110.50538) (width 0.25) (layer F.Cu) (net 10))
 (segment (start 149.8092 110.21314) (end 150.18512 109.83722) (width 0.25) (layer F.Cu) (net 10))
 (segment (start 149.8092 110.2233) (end 149.8092 110.21314) (width 0.25) (layer F.Cu) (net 10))
 (segment (start 150.13178 106.436998) (end 150.13178 109.78388) (width 0.25) (layer B.Cu) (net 10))
 (segment (start 150.759998 105.80878) (end 150.13178 106.436998) (width 0.25) (layer B.Cu) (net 10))
 (segment (start 150.13178 109.78388) (end 150.18512 109.83722) (width 0.25) (layer B.Cu) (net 10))
 (segment (start 152.92578 105.80878) (end 150.759998 105.80878) (width 0.25) (layer B.Cu) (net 10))
 (segment (start 153.38806 106.27106) (end 152.92578 105.80878) (width 0.25) (layer B.Cu) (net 10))
 (segment (start 153.38806 107.10672) (end 153.38806 106.27106) (width 0.25) (layer B.Cu) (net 10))
 (via (at 161.00552 110.42396) (size 0.8) (drill 0.4) (layers F.Cu B.Cu) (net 6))
 (segment (start 151.153044 109.10672) (end 151.38806 109.10672) (width 0.25) (layer F.Cu) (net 6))
 (segment (start 152.146019 110.632221) (end 149.738061 110.632221) (width 0.4) (layer B.Cu) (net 6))
 (segment (start 152.14854 110.6297) (end 152.146019 110.632221) (width 0.4) (layer B.Cu) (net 6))
 (segment (start 149.738061 110.632221) (end 148.72208 109.61624) (width 0.4) (layer B.Cu) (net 6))
 (segment (start 148.72208 109.61624) (end 148.72208 106.9975) (width 0.4) (layer B.Cu) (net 6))
 (segment (start 150.950061 105.232861) (end 151.54148 104.641442) (width 0.4) (layer B.Cu) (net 6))
 (segment (start 150.080319 105.232861) (end 150.950061 105.232861) (width 0.4) (layer B.Cu) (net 6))
 (segment (start 148.72208 106.5911) (end 150.080319 105.232861) (width 0.4) (layer B.Cu) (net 6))
 (segment (start 148.72208 106.9975) (end 148.72208 106.5911) (width 0.4) (layer B.Cu) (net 6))
 (segment (start 151.54148 104.641442) (end 153.69032 104.52354) (width 0.4) (layer B.Cu) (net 6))
 (segment (start 153.69032 104.52354) (end 153.630422 104.641442) (width 0.4) (layer B.Cu) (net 6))
 (via (at 153.69032 104.52354) (size 0.8) (drill 0.4) (layers F.Cu B.Cu) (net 6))
 (segment (start 153.69032 103.75138) (end 153.69032 104.52354) (width 0.4) (layer F.Cu) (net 6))
 (segment (start 153.69032 104.52354) (end 153.89098 104.7242) (width 0.4) (layer B.Cu) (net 6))
 (segment (start 153.89098 104.7242) (end 157.46984 104.7242) (width 0.4) (layer B.Cu) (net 6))
 (segment (start 157.46984 104.7242) (end 157.46984 104.76484) (width 0.4) (layer B.Cu) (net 6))
 (segment (start 157.46984 104.76484) (end 157.74162 105.03662) (width 0.4) (layer B.Cu) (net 6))
 (segment (start 157.74162 105.03662) (end 157.74162 105.03662) (width 0.4) (layer B.Cu) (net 6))
 (via (at 157.74162 105.03662) (size 0.8) (drill 0.4) (layers F.Cu B.Cu) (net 6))
 (segment (start 157.36062 104.65562) (end 157.74162 105.03662) (width 0.4) (layer F.Cu) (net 6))
 (segment (start 157.36062 102.62334) (end 157.36062 104.65562) (width 0.4) (layer F.Cu) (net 6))
 (segment (start 159.301561 105.436619) (end 160.6169 106.751958) (width 0.4) (layer B.Cu) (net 6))
 (segment (start 158.141619 105.436619) (end 159.301561 105.436619) (width 0.4) (layer B.Cu) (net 6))
 (segment (start 157.74162 105.03662) (end 158.141619 105.436619) (width 0.4) (layer B.Cu) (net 6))
 (segment (start 160.6169 110.03534) (end 161.00552 110.42396) (width 0.4) (layer B.Cu) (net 6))
 (segment (start 160.6169 106.751958) (end 160.6169 110.03534) (width 0.4) (layer B.Cu) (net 6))
 (segment (start 161.013836 110.432276) (end 161.00552 110.42396) (width 0.4) (layer F.Cu) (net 6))
 (segment (start 161.30792 110.432276) (end 161.013836 110.432276) (width 0.4) (layer F.Cu) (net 6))
 (segment (start 151.38806 109.86922) (end 152.14854 110.6297) (width 0.4) (layer F.Cu) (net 6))
 (segment (start 151.38806 109.10672) (end 151.38806 109.86922) (width 0.4) (layer F.Cu) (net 6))
 (segment (start 146.94796 109.574678) (end 147.67306 108.849578) (width 0.4) (layer F.Cu) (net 6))
 (segment (start 147.67306 108.849578) (end 147.67306 108.15574) (width 0.4) (layer F.Cu) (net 6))
 (segment (start 147.67306 108.15574) (end 147.79498 108.03382) (width 0.4) (layer F.Cu) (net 6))
 (segment (start 150.458061 108.176721) (end 151.38806 109.10672) (width 0.4) (layer F.Cu) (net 6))
 (segment (start 147.937881 108.176721) (end 150.458061 108.176721) (width 0.4) (layer F.Cu) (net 6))
 (segment (start 147.79498 108.03382) (end 147.937881 108.176721) (width 0.4) (layer F.Cu) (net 6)))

